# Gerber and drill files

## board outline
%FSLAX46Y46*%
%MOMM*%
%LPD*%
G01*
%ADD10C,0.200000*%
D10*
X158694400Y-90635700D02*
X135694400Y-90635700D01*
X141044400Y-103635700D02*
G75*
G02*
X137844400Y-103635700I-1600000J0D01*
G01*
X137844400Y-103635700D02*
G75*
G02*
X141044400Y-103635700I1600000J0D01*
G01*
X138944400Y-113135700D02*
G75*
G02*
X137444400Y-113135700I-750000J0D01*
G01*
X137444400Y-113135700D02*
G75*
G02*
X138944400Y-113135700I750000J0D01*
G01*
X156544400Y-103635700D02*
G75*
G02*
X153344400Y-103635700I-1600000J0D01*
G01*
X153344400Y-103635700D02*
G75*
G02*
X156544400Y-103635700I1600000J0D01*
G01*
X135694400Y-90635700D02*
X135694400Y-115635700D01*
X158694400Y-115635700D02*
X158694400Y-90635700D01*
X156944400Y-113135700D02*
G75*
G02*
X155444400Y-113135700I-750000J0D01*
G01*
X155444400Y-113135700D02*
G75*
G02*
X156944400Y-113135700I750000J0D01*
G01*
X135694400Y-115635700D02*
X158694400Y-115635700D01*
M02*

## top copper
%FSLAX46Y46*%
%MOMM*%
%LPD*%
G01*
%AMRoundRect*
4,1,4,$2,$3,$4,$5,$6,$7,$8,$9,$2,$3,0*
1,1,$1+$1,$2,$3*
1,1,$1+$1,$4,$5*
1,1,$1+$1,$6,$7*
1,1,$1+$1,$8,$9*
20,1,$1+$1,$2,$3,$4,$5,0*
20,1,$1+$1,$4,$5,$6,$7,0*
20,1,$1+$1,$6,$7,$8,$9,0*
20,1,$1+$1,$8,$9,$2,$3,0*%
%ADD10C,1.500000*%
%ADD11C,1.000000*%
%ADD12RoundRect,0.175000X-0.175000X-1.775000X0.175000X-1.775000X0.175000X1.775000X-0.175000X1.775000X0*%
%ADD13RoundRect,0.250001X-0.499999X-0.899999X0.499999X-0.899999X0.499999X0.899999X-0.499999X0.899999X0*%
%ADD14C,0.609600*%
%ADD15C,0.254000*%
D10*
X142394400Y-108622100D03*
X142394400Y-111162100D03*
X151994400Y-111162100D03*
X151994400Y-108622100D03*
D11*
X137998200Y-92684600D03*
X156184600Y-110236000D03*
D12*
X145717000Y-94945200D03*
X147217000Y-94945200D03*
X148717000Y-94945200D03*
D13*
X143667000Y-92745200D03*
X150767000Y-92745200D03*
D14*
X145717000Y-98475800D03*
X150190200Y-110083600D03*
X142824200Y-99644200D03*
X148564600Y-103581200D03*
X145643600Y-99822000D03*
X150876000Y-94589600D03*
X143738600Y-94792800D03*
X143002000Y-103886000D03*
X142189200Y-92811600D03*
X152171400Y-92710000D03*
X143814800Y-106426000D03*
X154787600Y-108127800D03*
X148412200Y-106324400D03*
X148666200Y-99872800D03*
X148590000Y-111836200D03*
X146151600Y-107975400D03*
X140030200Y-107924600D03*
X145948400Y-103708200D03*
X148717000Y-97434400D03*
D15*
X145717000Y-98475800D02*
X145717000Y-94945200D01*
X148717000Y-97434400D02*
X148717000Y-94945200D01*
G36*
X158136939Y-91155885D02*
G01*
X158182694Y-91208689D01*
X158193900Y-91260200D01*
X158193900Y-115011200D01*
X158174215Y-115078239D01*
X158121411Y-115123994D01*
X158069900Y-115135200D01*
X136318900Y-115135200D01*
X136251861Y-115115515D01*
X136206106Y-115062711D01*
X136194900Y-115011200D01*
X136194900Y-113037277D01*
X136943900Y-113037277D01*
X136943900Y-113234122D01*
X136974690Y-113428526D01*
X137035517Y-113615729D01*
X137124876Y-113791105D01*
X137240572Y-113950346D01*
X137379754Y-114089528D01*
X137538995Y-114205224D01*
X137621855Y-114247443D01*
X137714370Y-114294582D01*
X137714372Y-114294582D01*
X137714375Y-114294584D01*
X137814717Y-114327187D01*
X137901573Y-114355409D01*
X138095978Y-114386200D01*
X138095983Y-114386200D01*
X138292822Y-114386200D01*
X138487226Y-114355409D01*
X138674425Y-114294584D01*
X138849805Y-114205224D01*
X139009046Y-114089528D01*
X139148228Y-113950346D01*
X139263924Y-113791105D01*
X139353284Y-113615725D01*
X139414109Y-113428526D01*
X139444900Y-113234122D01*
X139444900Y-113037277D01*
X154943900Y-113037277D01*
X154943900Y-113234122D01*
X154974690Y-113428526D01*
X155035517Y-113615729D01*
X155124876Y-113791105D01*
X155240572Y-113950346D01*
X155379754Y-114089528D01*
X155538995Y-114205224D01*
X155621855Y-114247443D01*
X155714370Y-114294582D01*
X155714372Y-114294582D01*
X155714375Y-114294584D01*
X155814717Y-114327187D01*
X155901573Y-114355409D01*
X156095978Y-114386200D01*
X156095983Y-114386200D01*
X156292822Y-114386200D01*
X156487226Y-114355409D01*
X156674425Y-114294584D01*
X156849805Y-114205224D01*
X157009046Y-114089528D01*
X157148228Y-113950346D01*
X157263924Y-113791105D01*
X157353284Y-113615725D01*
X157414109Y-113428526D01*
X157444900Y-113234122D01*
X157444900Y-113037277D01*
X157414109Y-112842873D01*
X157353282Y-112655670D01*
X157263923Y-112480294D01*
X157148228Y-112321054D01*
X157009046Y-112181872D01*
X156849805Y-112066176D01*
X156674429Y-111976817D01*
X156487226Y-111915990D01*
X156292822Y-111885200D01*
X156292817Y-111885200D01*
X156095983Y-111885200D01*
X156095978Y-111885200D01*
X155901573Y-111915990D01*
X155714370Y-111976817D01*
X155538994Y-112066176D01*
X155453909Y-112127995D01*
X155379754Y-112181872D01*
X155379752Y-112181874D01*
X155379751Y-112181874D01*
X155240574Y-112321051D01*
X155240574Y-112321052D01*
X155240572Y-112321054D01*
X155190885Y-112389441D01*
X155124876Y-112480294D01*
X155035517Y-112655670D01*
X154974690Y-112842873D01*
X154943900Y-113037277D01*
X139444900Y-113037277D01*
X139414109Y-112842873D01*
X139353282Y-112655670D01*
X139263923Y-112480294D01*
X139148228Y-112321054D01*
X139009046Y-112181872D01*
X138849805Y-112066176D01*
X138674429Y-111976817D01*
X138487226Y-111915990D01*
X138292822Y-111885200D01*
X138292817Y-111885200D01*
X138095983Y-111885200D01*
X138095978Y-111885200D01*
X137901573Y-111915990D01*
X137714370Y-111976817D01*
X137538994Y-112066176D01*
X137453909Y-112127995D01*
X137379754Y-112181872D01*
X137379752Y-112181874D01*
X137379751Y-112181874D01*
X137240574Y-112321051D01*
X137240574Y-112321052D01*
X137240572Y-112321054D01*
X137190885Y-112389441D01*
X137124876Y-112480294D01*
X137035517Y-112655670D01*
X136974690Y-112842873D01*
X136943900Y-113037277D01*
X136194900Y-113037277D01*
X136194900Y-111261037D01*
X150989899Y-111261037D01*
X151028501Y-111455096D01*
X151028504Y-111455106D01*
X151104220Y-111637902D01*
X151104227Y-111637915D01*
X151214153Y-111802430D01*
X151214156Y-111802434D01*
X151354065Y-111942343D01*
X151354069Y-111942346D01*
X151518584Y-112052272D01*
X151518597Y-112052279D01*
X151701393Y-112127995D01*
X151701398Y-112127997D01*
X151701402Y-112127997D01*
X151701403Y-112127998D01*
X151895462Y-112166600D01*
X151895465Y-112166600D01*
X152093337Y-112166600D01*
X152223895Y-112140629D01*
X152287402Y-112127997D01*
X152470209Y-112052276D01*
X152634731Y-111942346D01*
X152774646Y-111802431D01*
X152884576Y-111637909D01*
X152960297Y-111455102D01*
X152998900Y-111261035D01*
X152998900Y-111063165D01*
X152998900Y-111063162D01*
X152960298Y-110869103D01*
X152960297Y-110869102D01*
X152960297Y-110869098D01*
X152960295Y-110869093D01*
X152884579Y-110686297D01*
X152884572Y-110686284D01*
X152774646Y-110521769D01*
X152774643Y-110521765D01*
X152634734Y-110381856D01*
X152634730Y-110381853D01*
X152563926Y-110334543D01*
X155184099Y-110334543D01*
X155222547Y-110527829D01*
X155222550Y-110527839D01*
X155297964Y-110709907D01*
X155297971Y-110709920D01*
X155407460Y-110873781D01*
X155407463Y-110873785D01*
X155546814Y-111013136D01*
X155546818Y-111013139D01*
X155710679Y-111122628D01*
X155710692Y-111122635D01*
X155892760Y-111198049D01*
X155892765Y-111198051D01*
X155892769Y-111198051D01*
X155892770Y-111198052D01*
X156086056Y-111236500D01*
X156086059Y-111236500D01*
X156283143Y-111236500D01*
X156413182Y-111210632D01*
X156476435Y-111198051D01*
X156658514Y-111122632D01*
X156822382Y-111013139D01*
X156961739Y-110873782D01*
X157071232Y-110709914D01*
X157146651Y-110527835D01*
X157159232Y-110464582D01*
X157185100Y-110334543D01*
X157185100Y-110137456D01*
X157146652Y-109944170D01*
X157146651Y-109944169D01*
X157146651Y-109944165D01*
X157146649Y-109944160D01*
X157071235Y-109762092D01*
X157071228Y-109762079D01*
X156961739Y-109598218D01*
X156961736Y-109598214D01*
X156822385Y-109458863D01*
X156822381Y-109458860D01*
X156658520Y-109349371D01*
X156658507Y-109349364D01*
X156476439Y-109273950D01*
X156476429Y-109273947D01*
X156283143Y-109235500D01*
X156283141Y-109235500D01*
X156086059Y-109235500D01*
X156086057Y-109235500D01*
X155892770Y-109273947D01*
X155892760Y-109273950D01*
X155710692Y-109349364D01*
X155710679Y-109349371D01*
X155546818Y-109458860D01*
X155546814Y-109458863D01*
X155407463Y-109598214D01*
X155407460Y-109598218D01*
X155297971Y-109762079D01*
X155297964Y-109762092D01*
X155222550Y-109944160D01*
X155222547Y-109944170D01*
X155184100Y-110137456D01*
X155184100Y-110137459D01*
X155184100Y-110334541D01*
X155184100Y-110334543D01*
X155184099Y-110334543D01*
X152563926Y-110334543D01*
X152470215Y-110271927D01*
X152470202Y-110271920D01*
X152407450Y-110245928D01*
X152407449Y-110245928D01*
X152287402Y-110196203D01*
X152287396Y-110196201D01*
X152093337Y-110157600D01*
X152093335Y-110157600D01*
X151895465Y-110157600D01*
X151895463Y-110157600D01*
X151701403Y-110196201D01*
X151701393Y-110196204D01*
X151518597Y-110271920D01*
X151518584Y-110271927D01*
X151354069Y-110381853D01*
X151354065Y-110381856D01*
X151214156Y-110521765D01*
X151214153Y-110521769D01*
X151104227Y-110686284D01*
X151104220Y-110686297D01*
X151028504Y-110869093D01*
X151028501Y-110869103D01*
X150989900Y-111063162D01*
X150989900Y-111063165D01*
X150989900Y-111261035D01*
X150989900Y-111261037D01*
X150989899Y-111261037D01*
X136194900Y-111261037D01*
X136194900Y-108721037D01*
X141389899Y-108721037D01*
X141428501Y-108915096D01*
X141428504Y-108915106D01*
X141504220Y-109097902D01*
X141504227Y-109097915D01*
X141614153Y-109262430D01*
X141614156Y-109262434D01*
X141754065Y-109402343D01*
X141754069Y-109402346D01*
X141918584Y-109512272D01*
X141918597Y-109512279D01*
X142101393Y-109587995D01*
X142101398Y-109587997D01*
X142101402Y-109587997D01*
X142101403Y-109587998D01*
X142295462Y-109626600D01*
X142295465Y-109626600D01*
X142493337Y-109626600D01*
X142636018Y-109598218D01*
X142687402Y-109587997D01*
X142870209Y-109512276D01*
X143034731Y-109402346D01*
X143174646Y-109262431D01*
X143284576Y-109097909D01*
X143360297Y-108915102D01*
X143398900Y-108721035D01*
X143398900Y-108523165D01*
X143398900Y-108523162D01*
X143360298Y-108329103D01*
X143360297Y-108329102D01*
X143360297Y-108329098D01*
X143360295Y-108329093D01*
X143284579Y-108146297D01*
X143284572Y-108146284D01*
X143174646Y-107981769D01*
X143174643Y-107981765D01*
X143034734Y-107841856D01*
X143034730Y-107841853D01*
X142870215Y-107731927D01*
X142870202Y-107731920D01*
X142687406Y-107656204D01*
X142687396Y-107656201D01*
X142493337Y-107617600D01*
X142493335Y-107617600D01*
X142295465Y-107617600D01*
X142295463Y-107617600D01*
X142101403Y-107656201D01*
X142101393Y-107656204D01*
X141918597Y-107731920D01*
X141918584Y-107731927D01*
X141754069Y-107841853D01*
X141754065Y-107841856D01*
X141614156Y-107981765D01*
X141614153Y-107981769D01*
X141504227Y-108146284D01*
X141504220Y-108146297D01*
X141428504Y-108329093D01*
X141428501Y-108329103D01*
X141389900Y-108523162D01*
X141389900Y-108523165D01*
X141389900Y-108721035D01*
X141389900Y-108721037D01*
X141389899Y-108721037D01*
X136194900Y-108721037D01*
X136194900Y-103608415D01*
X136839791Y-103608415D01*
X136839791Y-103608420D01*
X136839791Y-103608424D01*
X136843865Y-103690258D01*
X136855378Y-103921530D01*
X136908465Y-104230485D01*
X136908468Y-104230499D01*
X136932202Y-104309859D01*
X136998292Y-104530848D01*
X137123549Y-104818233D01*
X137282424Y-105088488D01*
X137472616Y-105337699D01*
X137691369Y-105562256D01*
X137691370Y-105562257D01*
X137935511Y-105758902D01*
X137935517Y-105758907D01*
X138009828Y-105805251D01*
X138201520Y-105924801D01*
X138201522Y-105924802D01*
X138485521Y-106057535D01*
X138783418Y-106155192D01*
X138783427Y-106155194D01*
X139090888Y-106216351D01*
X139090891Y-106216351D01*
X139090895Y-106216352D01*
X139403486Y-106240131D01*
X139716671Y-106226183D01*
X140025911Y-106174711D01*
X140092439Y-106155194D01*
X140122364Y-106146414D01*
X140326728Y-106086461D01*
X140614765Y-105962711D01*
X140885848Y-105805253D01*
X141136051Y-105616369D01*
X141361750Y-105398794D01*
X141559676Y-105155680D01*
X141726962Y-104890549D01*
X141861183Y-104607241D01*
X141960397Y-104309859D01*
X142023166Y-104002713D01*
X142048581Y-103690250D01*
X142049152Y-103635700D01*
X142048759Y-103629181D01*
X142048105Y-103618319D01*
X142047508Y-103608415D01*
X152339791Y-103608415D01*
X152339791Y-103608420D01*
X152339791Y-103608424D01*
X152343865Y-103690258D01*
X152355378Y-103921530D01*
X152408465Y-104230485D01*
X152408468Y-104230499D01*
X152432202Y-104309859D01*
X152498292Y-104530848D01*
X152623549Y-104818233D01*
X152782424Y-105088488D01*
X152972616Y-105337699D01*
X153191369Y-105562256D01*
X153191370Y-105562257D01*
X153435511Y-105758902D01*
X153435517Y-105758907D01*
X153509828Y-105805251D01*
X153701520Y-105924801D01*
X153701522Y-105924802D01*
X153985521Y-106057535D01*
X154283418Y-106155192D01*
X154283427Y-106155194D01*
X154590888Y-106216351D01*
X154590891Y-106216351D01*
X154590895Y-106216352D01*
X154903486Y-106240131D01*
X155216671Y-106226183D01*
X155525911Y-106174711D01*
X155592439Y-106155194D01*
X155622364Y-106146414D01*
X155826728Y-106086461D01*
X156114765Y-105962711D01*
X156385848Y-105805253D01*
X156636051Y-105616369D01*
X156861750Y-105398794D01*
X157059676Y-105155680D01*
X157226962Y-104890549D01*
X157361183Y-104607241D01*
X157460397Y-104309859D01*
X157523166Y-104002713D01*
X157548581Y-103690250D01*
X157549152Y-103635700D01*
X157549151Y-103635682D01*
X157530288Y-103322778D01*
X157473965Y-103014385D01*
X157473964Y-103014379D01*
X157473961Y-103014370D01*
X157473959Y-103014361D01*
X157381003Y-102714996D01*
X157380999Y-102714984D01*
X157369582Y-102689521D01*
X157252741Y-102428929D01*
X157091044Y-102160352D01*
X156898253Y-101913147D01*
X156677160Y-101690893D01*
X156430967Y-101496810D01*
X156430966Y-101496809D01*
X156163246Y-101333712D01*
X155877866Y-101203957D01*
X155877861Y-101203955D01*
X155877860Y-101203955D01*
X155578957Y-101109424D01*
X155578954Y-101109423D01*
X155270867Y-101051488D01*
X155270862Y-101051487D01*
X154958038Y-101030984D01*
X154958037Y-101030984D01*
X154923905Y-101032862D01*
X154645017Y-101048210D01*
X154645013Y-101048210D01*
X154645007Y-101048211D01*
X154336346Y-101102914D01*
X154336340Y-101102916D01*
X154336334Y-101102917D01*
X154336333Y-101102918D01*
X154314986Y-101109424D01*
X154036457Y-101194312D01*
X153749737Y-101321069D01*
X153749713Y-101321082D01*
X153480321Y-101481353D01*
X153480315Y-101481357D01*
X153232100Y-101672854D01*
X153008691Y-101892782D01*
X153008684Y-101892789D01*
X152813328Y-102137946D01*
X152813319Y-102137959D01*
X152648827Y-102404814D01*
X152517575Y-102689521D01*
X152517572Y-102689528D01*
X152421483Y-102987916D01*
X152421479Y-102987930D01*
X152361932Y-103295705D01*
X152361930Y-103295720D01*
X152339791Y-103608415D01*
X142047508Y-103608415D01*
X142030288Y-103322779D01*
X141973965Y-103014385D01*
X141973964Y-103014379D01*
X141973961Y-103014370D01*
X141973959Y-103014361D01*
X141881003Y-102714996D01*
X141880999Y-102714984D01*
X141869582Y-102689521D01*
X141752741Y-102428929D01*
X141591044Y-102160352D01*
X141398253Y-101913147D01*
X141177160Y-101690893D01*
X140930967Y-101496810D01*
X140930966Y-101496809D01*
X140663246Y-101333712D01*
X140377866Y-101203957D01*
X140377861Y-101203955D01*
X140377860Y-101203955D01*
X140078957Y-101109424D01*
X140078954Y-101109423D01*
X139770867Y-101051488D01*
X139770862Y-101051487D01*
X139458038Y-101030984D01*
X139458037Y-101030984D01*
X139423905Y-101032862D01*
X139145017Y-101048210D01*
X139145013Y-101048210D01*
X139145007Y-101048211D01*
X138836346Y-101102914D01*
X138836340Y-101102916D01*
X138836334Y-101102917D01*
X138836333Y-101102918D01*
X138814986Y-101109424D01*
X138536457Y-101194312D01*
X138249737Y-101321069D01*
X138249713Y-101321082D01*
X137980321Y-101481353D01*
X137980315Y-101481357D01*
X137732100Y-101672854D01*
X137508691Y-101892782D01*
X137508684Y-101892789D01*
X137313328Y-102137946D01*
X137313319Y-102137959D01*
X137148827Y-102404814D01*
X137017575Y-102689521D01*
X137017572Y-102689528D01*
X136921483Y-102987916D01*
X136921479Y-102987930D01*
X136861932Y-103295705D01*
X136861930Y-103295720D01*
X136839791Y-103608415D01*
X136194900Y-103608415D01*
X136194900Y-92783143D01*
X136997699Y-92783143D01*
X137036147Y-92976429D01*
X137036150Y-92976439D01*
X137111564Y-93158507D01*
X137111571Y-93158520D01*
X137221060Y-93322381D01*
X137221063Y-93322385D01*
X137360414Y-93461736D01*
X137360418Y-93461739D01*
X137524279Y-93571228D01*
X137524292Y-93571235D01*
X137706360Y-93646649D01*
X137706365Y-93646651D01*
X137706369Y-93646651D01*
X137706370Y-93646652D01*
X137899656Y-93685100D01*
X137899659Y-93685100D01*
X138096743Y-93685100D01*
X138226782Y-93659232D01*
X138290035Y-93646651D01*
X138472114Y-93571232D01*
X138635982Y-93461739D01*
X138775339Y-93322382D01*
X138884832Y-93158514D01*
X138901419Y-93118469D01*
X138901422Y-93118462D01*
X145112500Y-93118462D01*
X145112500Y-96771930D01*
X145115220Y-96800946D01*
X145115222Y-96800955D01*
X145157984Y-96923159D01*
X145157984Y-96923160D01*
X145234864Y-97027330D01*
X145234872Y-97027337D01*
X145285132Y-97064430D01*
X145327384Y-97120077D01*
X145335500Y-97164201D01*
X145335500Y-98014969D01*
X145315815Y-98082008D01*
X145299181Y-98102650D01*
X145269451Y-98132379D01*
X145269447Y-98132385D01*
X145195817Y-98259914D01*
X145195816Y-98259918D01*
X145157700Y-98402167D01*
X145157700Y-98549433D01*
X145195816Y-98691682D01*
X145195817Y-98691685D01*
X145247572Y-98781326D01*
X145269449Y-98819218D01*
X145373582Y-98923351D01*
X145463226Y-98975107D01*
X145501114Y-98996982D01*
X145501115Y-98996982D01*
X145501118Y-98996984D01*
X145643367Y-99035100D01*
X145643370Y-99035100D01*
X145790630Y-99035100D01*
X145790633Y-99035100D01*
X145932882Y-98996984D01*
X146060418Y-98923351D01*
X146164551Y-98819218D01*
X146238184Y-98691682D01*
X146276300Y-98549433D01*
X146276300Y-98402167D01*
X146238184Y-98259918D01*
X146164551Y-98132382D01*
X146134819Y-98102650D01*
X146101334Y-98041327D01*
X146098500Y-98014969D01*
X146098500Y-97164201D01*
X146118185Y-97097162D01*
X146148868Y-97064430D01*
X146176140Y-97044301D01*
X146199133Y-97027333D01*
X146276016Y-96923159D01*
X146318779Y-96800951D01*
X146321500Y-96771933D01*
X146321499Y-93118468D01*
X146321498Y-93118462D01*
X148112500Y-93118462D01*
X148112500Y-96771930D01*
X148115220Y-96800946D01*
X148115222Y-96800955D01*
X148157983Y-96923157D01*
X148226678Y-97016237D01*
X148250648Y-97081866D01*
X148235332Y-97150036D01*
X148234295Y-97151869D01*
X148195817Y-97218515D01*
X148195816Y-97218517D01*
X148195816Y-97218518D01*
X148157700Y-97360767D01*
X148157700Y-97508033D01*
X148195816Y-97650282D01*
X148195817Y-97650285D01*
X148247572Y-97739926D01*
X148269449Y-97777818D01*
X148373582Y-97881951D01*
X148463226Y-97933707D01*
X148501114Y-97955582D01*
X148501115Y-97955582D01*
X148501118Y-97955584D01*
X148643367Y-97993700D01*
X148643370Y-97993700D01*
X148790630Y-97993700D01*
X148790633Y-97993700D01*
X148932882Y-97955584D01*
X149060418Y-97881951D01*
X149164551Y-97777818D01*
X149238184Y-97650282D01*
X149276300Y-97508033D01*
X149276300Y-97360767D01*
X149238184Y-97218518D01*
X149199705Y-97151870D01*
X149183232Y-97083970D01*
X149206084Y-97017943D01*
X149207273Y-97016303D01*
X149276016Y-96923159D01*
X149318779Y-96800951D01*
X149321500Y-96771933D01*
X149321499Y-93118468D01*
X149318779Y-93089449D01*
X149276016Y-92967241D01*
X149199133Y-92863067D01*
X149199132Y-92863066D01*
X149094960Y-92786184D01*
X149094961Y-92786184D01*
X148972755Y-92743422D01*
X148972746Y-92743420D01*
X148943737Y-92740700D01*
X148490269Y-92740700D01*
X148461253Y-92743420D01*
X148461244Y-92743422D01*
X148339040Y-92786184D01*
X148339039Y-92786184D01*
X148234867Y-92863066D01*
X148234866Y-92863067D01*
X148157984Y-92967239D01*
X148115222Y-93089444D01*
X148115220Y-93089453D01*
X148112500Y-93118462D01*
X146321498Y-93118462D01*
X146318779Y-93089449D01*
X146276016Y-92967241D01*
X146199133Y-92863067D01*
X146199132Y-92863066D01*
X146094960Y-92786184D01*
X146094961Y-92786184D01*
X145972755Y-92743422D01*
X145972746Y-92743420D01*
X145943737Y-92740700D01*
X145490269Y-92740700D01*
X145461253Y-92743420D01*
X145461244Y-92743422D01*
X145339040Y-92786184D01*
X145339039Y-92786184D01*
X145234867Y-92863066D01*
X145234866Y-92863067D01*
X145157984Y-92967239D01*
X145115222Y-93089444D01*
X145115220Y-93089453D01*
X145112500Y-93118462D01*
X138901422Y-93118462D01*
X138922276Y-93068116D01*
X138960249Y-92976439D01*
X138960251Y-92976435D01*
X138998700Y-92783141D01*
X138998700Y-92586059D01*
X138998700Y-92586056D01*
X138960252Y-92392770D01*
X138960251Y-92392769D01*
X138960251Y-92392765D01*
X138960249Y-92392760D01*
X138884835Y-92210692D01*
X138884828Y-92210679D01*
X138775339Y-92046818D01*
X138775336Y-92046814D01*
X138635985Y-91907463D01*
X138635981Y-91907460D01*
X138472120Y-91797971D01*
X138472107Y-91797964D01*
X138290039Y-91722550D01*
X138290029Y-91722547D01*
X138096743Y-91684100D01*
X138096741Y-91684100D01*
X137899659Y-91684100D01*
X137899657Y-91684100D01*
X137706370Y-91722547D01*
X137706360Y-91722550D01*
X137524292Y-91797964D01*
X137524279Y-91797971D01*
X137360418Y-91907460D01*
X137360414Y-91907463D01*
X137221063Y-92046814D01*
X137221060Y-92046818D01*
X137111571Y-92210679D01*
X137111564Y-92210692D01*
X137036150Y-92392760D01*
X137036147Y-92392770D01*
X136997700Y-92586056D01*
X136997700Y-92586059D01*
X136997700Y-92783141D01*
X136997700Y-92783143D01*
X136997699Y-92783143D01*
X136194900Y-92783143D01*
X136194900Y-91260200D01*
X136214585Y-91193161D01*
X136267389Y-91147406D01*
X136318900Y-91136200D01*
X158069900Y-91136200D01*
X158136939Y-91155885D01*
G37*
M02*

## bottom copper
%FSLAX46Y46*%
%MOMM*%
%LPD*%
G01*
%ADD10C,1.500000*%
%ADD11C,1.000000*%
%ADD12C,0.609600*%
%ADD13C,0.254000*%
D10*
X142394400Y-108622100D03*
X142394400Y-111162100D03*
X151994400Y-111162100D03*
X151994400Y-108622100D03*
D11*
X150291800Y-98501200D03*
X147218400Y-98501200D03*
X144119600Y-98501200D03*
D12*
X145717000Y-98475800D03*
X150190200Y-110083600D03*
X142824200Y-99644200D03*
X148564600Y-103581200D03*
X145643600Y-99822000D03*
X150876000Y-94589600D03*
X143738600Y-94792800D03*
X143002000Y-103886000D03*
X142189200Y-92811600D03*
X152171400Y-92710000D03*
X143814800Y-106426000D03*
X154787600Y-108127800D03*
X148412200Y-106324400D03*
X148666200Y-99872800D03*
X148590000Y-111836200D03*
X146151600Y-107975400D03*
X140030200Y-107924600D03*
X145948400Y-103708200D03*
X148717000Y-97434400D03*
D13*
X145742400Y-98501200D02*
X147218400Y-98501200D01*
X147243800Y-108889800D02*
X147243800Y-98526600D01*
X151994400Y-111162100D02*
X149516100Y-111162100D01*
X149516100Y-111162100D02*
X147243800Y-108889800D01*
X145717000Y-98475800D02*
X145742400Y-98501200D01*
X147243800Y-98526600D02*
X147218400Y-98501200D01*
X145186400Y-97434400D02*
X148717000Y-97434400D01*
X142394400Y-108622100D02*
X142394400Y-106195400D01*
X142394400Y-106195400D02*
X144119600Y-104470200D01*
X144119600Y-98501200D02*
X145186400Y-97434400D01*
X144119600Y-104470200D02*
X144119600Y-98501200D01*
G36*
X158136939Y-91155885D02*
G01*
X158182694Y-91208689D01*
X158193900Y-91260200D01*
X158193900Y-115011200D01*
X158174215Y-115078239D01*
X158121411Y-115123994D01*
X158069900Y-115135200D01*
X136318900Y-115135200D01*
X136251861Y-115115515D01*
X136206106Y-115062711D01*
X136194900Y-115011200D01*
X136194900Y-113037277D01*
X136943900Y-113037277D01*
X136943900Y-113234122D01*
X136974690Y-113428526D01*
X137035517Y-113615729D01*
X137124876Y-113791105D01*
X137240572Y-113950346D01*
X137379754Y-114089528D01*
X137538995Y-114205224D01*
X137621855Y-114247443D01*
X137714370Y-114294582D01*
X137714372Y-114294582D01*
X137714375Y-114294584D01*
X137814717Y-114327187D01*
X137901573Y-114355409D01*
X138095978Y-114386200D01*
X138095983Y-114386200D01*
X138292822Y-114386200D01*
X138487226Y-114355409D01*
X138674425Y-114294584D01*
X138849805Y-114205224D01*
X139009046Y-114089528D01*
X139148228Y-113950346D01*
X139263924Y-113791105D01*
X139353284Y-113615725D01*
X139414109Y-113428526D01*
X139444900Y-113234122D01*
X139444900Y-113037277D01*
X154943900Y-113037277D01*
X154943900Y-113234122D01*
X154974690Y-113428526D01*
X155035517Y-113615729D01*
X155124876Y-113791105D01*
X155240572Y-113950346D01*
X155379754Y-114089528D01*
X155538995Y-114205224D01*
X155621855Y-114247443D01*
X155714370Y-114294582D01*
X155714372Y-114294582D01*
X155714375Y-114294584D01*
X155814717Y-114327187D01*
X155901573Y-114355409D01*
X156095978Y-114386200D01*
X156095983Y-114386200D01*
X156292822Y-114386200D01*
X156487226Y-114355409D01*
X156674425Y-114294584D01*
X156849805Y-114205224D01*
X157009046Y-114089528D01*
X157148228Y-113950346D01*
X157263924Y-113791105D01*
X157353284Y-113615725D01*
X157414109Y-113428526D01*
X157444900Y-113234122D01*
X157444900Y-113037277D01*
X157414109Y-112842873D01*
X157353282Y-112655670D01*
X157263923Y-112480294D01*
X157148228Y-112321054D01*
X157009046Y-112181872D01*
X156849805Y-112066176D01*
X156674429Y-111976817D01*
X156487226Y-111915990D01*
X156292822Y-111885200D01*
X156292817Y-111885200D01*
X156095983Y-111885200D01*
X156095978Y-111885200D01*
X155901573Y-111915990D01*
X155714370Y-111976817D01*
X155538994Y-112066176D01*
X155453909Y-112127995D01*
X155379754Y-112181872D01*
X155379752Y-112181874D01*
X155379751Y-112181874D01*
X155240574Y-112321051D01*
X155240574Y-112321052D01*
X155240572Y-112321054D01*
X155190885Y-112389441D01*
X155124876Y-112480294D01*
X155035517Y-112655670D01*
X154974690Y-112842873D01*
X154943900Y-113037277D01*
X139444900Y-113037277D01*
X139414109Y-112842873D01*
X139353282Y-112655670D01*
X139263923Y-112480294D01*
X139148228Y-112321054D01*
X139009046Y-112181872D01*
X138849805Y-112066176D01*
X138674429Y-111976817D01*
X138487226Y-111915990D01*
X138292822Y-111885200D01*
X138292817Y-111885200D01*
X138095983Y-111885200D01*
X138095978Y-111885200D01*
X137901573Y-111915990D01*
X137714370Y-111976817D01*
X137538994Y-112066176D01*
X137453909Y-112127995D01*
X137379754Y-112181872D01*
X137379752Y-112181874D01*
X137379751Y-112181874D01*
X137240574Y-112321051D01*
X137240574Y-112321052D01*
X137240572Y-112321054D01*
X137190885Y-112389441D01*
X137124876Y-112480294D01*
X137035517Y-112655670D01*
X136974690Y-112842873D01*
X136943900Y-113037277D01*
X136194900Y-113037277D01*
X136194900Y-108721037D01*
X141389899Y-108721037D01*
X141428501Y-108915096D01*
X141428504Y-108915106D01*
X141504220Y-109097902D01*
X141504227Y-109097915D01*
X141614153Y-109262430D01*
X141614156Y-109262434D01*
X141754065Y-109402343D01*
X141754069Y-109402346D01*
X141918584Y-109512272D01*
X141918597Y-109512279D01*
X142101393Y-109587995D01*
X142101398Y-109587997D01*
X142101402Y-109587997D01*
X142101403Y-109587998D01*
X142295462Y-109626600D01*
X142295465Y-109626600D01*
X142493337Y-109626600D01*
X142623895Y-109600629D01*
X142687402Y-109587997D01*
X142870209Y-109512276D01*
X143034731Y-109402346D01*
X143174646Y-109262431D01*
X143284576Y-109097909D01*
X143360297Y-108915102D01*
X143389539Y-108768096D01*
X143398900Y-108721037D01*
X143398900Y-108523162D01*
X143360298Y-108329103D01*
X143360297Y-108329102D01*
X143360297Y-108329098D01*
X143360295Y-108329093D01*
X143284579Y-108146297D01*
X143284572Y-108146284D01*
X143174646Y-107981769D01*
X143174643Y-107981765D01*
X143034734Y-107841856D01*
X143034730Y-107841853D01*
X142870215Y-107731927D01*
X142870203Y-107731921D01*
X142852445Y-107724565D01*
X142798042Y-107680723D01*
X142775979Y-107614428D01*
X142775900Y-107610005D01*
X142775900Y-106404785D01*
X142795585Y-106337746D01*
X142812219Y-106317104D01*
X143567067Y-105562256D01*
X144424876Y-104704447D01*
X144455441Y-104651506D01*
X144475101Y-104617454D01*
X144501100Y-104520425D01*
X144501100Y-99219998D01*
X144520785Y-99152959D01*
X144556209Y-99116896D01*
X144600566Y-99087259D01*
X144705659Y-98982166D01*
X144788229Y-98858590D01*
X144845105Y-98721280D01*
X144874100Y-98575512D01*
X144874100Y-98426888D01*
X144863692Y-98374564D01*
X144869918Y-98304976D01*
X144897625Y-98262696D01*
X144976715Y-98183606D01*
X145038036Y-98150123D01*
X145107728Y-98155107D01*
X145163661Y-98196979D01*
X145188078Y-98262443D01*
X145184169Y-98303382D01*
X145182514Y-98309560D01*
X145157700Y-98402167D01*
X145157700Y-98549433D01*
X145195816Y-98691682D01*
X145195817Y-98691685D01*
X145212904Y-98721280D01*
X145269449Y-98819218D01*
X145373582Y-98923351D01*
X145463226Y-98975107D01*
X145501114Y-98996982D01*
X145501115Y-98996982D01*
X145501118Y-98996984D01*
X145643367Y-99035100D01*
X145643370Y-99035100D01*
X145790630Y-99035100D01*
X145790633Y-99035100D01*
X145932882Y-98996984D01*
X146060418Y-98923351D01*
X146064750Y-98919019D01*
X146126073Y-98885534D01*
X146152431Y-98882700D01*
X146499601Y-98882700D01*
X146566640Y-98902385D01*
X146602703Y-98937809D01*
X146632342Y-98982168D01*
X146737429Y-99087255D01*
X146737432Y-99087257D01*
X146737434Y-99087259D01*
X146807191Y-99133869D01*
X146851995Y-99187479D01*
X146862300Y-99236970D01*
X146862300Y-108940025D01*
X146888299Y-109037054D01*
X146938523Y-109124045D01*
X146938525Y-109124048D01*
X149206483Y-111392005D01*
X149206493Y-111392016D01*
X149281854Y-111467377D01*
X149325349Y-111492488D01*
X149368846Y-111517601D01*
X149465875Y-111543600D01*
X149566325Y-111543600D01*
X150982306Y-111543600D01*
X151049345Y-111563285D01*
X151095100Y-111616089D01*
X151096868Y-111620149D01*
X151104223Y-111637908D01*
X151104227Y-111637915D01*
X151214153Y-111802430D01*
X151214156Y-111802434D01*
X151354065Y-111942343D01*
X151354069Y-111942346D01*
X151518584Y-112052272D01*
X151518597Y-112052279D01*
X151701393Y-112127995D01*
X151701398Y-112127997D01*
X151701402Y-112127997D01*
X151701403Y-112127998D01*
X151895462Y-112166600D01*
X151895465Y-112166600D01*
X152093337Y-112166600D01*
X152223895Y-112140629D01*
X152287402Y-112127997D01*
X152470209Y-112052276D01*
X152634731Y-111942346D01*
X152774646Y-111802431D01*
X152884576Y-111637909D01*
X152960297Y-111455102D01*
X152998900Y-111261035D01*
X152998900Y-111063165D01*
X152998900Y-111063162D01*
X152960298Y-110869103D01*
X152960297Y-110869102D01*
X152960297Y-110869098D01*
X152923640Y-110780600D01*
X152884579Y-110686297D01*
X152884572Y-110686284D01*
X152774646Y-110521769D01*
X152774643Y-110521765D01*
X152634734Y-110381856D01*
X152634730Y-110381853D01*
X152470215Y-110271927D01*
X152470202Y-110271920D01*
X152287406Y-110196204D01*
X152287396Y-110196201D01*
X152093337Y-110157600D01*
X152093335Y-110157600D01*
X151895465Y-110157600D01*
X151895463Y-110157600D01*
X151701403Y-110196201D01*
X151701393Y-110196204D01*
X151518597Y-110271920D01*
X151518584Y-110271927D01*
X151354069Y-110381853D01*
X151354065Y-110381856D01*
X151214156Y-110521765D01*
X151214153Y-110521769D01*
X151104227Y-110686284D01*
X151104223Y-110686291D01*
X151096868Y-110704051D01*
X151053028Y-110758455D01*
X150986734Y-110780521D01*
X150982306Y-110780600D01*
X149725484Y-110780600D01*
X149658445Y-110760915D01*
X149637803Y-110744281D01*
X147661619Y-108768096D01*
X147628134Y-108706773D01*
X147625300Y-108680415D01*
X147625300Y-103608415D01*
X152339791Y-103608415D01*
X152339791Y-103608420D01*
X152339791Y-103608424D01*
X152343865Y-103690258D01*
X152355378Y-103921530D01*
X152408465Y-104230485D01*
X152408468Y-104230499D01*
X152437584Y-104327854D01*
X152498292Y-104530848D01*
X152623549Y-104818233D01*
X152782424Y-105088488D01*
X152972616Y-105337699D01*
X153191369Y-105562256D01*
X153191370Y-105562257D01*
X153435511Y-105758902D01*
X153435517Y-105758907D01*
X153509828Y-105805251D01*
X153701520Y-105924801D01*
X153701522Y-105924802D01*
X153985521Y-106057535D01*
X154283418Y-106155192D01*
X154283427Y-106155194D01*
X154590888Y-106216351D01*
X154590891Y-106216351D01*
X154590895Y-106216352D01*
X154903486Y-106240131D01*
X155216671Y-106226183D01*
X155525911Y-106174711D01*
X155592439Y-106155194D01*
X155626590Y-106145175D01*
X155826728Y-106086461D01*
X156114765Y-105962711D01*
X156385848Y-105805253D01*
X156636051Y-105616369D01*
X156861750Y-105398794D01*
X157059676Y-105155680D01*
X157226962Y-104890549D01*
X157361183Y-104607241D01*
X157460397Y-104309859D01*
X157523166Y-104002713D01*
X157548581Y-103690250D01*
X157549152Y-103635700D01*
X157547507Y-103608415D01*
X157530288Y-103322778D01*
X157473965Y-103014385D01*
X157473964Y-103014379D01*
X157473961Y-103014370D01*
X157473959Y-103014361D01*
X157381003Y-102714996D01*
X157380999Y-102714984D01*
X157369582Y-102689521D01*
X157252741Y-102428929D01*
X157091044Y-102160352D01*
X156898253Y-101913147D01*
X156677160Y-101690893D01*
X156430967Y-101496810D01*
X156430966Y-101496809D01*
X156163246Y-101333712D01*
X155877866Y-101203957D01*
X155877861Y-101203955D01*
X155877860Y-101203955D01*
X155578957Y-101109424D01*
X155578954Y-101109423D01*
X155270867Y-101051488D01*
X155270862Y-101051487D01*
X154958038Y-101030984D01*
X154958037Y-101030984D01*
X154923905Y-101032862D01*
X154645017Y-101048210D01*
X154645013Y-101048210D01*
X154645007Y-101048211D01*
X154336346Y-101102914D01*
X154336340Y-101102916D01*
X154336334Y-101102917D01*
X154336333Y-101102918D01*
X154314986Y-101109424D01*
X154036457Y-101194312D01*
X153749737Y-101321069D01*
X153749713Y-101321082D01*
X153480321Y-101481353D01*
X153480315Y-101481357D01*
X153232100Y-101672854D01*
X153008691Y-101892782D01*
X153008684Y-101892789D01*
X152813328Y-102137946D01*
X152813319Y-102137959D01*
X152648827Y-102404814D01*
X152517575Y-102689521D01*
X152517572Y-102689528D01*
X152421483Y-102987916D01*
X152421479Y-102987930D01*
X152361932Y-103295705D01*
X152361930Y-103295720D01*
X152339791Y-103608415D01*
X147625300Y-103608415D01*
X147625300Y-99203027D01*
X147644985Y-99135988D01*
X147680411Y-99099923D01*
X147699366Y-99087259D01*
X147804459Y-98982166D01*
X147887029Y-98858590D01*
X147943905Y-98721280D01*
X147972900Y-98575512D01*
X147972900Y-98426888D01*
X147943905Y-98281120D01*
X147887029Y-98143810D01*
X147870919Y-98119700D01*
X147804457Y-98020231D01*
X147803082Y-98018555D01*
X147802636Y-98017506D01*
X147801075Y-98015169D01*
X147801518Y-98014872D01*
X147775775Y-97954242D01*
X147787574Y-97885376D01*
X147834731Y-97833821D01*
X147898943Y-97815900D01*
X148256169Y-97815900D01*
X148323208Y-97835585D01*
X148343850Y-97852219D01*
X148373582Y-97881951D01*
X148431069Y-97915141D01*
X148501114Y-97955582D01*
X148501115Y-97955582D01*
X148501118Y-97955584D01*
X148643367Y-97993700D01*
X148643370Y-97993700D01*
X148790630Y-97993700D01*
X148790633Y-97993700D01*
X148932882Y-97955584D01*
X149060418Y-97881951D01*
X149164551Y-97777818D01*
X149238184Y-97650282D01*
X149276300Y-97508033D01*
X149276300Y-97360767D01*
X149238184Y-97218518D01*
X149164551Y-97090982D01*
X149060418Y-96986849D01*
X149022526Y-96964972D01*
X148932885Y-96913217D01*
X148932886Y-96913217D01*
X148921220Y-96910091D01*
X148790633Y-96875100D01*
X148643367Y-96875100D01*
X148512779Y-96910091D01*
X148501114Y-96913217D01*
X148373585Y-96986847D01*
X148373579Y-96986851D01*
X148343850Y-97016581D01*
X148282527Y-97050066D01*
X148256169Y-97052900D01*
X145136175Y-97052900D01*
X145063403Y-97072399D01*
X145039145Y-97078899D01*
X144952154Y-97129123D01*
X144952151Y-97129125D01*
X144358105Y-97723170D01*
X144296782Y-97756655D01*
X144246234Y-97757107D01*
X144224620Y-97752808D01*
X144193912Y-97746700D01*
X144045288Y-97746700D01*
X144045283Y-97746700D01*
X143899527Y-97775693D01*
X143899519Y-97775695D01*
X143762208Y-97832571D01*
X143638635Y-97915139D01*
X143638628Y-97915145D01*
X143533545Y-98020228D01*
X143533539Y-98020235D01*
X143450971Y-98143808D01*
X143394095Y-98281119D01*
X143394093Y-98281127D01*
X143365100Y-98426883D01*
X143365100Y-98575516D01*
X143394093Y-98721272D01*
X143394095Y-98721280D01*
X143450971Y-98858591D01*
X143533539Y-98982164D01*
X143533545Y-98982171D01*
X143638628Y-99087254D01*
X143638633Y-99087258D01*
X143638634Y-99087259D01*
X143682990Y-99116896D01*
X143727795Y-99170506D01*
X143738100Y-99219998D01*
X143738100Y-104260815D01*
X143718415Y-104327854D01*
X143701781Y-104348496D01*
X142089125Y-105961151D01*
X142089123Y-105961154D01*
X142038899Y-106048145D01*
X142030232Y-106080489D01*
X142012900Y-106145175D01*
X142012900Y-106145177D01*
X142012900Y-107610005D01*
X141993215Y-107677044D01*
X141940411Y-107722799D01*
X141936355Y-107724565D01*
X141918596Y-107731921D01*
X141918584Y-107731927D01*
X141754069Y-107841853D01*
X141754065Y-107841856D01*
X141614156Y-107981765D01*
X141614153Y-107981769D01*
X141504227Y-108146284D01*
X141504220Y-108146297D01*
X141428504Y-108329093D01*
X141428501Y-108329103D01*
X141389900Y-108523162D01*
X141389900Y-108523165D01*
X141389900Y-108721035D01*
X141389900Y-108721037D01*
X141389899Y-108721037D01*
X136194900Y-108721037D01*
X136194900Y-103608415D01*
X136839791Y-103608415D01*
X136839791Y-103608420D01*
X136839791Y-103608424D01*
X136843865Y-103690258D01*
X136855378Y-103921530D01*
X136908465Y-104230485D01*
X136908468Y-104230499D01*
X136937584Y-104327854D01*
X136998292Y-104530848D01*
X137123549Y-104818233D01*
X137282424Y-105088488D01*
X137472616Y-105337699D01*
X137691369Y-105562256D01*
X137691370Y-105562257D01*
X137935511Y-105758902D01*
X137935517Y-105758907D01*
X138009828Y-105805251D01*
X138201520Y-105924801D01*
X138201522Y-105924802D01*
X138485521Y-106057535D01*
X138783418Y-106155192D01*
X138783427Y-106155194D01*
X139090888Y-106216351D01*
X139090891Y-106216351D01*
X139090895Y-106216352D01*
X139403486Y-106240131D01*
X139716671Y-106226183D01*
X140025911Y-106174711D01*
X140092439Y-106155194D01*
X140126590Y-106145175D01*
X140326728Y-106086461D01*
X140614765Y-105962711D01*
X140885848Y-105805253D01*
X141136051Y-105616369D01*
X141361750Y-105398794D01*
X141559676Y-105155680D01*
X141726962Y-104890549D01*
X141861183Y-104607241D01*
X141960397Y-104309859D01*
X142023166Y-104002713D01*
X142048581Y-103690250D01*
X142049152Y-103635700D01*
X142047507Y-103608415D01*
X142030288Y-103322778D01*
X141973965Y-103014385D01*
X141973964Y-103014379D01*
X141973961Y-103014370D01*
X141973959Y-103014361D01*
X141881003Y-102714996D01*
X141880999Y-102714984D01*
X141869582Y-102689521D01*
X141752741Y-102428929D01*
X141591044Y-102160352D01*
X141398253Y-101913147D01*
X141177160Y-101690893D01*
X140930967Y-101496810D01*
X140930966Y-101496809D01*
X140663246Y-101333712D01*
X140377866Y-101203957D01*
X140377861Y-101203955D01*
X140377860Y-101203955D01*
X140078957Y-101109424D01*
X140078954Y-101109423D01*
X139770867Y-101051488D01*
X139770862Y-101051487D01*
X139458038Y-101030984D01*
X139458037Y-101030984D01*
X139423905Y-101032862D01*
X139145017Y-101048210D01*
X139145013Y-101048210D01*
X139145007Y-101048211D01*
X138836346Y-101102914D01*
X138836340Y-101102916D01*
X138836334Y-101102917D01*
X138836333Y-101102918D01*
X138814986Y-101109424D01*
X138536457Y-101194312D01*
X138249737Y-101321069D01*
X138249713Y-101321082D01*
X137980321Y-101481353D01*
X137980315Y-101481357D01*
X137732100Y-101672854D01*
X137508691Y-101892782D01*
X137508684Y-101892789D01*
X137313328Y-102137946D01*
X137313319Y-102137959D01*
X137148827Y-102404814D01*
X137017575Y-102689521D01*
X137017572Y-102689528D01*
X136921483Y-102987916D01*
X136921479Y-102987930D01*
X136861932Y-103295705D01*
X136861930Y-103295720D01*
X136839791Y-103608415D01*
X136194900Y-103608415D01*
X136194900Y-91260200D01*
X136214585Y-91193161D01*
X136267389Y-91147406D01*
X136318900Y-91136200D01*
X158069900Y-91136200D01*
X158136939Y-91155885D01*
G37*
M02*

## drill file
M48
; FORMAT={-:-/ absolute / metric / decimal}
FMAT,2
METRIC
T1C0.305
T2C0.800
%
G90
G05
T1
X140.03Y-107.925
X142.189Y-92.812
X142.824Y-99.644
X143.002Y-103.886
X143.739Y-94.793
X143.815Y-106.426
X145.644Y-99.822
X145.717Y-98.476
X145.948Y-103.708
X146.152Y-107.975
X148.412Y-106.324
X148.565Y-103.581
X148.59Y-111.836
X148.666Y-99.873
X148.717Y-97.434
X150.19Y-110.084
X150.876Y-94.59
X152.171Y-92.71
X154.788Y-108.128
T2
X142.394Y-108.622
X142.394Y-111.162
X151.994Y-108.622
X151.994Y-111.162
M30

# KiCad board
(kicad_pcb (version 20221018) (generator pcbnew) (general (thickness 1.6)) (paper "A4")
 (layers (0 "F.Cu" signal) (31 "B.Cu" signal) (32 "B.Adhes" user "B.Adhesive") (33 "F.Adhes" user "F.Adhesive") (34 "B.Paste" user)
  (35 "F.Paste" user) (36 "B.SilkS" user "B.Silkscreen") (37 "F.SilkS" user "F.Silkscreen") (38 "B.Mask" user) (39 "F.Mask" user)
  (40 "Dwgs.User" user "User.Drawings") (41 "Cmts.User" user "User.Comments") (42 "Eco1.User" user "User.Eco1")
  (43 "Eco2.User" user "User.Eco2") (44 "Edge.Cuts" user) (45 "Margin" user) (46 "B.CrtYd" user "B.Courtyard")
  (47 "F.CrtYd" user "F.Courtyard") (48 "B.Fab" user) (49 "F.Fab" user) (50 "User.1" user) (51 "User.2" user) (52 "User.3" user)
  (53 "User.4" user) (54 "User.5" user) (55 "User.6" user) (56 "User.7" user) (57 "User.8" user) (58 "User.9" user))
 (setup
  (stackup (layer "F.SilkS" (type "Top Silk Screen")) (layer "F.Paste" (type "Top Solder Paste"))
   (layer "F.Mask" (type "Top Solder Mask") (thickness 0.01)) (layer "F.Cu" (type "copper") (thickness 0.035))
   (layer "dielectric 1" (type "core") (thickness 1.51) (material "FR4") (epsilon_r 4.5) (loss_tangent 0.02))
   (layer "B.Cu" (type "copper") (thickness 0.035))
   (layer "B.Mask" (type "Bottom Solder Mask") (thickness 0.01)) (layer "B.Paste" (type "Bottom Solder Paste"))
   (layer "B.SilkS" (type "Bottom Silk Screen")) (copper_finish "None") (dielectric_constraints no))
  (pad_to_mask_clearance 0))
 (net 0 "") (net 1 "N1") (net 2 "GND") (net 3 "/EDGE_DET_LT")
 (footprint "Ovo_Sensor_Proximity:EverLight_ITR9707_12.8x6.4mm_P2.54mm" (layer "F.Cu") (at 147.1944 109.8921)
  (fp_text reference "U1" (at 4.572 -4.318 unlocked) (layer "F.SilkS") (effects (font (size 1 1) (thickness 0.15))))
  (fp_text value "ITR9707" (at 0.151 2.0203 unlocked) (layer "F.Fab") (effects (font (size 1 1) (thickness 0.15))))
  (pad "1" thru_hole circle (at -4.8 -1.27) (size 1.5 1.5) (drill 0.8) (layers "*.Cu" "*.Mask") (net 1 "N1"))
  (pad "2" thru_hole circle (at -4.8 1.27) (size 1.5 1.5) (drill 0.8) (layers "*.Cu" "*.Mask") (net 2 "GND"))
  (pad "3" thru_hole circle (at 4.8 1.27) (size 1.5 1.5) (drill 0.8) (layers "*.Cu" "*.Mask") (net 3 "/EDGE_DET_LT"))
  (pad "4" thru_hole circle (at 4.8 -1.27) (size 1.5 1.5) (drill 0.8) (layers "*.Cu" "*.Mask") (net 2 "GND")))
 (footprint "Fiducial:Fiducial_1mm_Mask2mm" (layer "F.Cu") (at 137.9982 92.6846)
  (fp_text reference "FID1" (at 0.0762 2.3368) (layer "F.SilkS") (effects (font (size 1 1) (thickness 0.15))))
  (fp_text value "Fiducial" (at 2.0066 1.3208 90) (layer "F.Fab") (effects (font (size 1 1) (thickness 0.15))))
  (pad "" smd circle (at 0 0) (size 1 1) (layers "F.Cu" "F.Mask") (solder_mask_margin 0.5) (clearance 0.5)))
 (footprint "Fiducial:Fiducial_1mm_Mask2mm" (layer "F.Cu") (at 156.1846 110.236)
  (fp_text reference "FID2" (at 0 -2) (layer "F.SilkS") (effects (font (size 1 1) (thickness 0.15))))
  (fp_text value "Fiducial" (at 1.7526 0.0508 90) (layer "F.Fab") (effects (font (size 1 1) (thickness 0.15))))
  (pad "" smd circle (at 0 0) (size 1 1) (layers "F.Cu" "F.Mask") (solder_mask_margin 0.5) (clearance 0.5)))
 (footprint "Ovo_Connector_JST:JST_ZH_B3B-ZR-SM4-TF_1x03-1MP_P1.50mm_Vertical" (layer "F.Cu") (at 147.217 94.2452)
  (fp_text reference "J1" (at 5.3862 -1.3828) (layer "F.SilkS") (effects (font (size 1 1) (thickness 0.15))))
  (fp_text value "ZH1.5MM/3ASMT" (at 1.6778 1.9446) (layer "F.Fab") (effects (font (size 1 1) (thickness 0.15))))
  (pad "1" smd roundrect (at -1.5 0.7) (size 0.7 3.9) (layers "F.Cu" "F.Paste" "F.Mask") (roundrect_rratio 0.25) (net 3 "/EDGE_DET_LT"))
  (pad "2" smd roundrect (at 0 0.7) (size 0.7 3.9) (layers "F.Cu" "F.Paste" "F.Mask") (roundrect_rratio 0.25) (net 2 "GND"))
  (pad "3" smd roundrect (at 1.5 0.7) (size 0.7 3.9) (layers "F.Cu" "F.Paste" "F.Mask") (roundrect_rratio 0.25) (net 1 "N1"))
  (pad "MP" smd roundrect (at -3.55 -1.5) (size 1.5 2.3) (layers "F.Cu" "F.Paste" "F.Mask") (roundrect_rratio 0.1666673333) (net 2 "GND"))
  (pad "MP" smd roundrect (at 3.55 -1.5) (size 1.5 2.3) (layers "F.Cu" "F.Paste" "F.Mask") (roundrect_rratio 0.1666673333) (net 2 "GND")))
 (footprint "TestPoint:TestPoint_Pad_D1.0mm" (layer "B.Cu") (at 150.2918 98.5012 180)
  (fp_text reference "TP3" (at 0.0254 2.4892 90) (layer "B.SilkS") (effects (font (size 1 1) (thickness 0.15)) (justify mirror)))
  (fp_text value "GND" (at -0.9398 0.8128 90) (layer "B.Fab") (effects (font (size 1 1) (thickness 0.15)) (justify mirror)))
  (pad "1" smd circle (at 0 0 180) (size 1 1) (layers "B.Cu" "B.Mask") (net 2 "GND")))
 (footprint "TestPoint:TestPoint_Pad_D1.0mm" (layer "B.Cu") (at 147.2184 98.5012 180)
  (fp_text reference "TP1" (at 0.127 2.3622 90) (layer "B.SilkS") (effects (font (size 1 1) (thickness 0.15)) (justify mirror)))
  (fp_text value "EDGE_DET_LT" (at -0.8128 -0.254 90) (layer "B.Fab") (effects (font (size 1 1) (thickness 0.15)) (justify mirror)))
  (pad "1" smd circle (at 0 0 180) (size 1 1) (layers "B.Cu" "B.Mask") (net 3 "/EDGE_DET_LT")))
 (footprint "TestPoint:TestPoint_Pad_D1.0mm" (layer "B.Cu") (at 144.1196 98.5012 180)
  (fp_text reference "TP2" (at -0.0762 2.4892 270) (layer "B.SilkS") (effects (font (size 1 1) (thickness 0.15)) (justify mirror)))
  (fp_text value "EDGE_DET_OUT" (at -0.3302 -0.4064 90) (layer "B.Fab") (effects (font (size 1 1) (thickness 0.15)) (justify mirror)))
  (pad "1" smd circle (at 0 0 180) (size 1 1) (layers "B.Cu" "B.Mask") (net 1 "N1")))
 (gr_line (start 158.6944 90.6357) (end 135.6944 90.6357) (stroke (width 0.2) (type solid)) (layer "Edge.Cuts"))
 (gr_circle (center 139.4444 103.6357) (end 141.0444 103.6357) (stroke (width 0.2) (type solid)) (fill none) (layer "Edge.Cuts"))
 (gr_circle (center 138.1944 113.1357) (end 138.9444 113.1357) (stroke (width 0.2) (type solid)) (fill none) (layer "Edge.Cuts"))
 (gr_circle (center 154.9444 103.6357) (end 156.5444 103.6357) (stroke (width 0.2) (type solid)) (fill none) (layer "Edge.Cuts"))
 (gr_line (start 135.6944 90.6357) (end 135.6944 115.6357) (stroke (width 0.2) (type solid)) (layer "Edge.Cuts"))
 (gr_line (start 158.6944 115.6357) (end 158.6944 90.6357) (stroke (width 0.2) (type solid)) (layer "Edge.Cuts"))
 (gr_circle (center 156.1944 113.1357) (end 156.9444 113.1357) (stroke (width 0.2) (type solid)) (fill none) (layer "Edge.Cuts"))
 (gr_line (start 135.6944 115.6357) (end 158.6944 115.6357) (stroke (width 0.2) (type solid)) (layer "Edge.Cuts"))
 (segment (start 145.717 98.4758) (end 145.717 94.9452) (width 0.254) (layer "F.Cu") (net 3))
 (via (at 145.717 98.4758) (size 0.6096) (drill 0.3048) (layers "F.Cu" "B.Cu") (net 3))
 (segment (start 145.7424 98.5012) (end 147.2184 98.5012) (width 0.254) (layer "B.Cu") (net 3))
 (segment (start 147.2438 108.8898) (end 147.2438 98.5266) (width 0.254) (layer "B.Cu") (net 3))
 (segment (start 151.9944 111.1621) (end 149.5161 111.1621) (width 0.254) (layer "B.Cu") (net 3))
 (segment (start 149.5161 111.1621) (end 147.2438 108.8898) (width 0.254) (layer "B.Cu") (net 3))
 (segment (start 145.717 98.4758) (end 145.7424 98.5012) (width 0.254) (layer "B.Cu") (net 3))
 (segment (start 147.2438 98.5266) (end 147.2184 98.5012) (width 0.254) (layer "B.Cu") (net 3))
 (via (at 150.1902 110.0836) (size 0.6096) (drill 0.3048) (layers "F.Cu" "B.Cu") (free) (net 2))
 (via (at 142.8242 99.6442) (size 0.6096) (drill 0.3048) (layers "F.Cu" "B.Cu") (free) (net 2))
 (via (at 148.5646 103.5812) (size 0.6096) (drill 0.3048) (layers "F.Cu" "B.Cu") (free) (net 2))
 (via (at 145.6436 99.822) (size 0.6096) (drill 0.3048) (layers "F.Cu" "B.Cu") (free) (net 2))
 (via (at 150.876 94.5896) (size 0.6096) (drill 0.3048) (layers "F.Cu" "B.Cu") (free) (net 2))
 (via (at 143.7386 94.7928) (size 0.6096) (drill 0.3048) (layers "F.Cu" "B.Cu") (free) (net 2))
 (via (at 143.002 103.886) (size 0.6096) (drill 0.3048) (layers "F.Cu" "B.Cu") (free) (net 2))
 (via (at 142.1892 92.8116) (size 0.6096) (drill 0.3048) (layers "F.Cu" "B.Cu") (free) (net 2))
 (via (at 152.1714 92.71) (size 0.6096) (drill 0.3048) (layers "F.Cu" "B.Cu") (free) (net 2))
 (via (at 143.8148 106.426) (size 0.6096) (drill 0.3048) (layers "F.Cu" "B.Cu") (free) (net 2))
 (via (at 154.7876 108.1278) (size 0.6096) (drill 0.3048) (layers "F.Cu" "B.Cu") (free) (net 2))
 (via (at 148.4122 106.3244) (size 0.6096) (drill 0.3048) (layers "F.Cu" "B.Cu") (free) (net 2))
 (via (at 148.6662 99.8728) (size 0.6096) (drill 0.3048) (layers "F.Cu" "B.Cu") (free) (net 2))
 (via (at 148.59 111.8362) (size 0.6096) (drill 0.3048) (layers "F.Cu" "B.Cu") (free) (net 2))
 (via (at 146.1516 107.9754) (size 0.6096) (drill 0.3048) (layers "F.Cu" "B.Cu") (free) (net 2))
 (via (at 140.0302 107.9246) (size 0.6096) (drill 0.3048) (layers "F.Cu" "B.Cu") (free) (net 2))
 (via (at 145.9484 103.7082) (size 0.6096) (drill 0.3048) (layers "F.Cu" "B.Cu") (free) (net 2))
 (segment (start 148.717 97.4344) (end 148.717 94.9452) (width 0.254) (layer "F.Cu") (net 1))
 (via (at 148.717 97.4344) (size 0.6096) (drill 0.3048) (layers "F.Cu" "B.Cu") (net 1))
 (segment (start 145.1864 97.4344) (end 148.717 97.4344) (width 0.254) (layer "B.Cu") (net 1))
 (segment (start 142.3944 108.6221) (end 142.3944 106.1954) (width 0.254) (layer "B.Cu") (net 1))
 (segment (start 142.3944 106.1954) (end 144.1196 104.4702) (width 0.254) (layer "B.Cu") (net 1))
 (segment (start 144.1196 98.5012) (end 145.1864 97.4344) (width 0.254) (layer "B.Cu") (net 1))
 (segment (start 144.1196 104.4702) (end 144.1196 98.5012) (width 0.254) (layer "B.Cu") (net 1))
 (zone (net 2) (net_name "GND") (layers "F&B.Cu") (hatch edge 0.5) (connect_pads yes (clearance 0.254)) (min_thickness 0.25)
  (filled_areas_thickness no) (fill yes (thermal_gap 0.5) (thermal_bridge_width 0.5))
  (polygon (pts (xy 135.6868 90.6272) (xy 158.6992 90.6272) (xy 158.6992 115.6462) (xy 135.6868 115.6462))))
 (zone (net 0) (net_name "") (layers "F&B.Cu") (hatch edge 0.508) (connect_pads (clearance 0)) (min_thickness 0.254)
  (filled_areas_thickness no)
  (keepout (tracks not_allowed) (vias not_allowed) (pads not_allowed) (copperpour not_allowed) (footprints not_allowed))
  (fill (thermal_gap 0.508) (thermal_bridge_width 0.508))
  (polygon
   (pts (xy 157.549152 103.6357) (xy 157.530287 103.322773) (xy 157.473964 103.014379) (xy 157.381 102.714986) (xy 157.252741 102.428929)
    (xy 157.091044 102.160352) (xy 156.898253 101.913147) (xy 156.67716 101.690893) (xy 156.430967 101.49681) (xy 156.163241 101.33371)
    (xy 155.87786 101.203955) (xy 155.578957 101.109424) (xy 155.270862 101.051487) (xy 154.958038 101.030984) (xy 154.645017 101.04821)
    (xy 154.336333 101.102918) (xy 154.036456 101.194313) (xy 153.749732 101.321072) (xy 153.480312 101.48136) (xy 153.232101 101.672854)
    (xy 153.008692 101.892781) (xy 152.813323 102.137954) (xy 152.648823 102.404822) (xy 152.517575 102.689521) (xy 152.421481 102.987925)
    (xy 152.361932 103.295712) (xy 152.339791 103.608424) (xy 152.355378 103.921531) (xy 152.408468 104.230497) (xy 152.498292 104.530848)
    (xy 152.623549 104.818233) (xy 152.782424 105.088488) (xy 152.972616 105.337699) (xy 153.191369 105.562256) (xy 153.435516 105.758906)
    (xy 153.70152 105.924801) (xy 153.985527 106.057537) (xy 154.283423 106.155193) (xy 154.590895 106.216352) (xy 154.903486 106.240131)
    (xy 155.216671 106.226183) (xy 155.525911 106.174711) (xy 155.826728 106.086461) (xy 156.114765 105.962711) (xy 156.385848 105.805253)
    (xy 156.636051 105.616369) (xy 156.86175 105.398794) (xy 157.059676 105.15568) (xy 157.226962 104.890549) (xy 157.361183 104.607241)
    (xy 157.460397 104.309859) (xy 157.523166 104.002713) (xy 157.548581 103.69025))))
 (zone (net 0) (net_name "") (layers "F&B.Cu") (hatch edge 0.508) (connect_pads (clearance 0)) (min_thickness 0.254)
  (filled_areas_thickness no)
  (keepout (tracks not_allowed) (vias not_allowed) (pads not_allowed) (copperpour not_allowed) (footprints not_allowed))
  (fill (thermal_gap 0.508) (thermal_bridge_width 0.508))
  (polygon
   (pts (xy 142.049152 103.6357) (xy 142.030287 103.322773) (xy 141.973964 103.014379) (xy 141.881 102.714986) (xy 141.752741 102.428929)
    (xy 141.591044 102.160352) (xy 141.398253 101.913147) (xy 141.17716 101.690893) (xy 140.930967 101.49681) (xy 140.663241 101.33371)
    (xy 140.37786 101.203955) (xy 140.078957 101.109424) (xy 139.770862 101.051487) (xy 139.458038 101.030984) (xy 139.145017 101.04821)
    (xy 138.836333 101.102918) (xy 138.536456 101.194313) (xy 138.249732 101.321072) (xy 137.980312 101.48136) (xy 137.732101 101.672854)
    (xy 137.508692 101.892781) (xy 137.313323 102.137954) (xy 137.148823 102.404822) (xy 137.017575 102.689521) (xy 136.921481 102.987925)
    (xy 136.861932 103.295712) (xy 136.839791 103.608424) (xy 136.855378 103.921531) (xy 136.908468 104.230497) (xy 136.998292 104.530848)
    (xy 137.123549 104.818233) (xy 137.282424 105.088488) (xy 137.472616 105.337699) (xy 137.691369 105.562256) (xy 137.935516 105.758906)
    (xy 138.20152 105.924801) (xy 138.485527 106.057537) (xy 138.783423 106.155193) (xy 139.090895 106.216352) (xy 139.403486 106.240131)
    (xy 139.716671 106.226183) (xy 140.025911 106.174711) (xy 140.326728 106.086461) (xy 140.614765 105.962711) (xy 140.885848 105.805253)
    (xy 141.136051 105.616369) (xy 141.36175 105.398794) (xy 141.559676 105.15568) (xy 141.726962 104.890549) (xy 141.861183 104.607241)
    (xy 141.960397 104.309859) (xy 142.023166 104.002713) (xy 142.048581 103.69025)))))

